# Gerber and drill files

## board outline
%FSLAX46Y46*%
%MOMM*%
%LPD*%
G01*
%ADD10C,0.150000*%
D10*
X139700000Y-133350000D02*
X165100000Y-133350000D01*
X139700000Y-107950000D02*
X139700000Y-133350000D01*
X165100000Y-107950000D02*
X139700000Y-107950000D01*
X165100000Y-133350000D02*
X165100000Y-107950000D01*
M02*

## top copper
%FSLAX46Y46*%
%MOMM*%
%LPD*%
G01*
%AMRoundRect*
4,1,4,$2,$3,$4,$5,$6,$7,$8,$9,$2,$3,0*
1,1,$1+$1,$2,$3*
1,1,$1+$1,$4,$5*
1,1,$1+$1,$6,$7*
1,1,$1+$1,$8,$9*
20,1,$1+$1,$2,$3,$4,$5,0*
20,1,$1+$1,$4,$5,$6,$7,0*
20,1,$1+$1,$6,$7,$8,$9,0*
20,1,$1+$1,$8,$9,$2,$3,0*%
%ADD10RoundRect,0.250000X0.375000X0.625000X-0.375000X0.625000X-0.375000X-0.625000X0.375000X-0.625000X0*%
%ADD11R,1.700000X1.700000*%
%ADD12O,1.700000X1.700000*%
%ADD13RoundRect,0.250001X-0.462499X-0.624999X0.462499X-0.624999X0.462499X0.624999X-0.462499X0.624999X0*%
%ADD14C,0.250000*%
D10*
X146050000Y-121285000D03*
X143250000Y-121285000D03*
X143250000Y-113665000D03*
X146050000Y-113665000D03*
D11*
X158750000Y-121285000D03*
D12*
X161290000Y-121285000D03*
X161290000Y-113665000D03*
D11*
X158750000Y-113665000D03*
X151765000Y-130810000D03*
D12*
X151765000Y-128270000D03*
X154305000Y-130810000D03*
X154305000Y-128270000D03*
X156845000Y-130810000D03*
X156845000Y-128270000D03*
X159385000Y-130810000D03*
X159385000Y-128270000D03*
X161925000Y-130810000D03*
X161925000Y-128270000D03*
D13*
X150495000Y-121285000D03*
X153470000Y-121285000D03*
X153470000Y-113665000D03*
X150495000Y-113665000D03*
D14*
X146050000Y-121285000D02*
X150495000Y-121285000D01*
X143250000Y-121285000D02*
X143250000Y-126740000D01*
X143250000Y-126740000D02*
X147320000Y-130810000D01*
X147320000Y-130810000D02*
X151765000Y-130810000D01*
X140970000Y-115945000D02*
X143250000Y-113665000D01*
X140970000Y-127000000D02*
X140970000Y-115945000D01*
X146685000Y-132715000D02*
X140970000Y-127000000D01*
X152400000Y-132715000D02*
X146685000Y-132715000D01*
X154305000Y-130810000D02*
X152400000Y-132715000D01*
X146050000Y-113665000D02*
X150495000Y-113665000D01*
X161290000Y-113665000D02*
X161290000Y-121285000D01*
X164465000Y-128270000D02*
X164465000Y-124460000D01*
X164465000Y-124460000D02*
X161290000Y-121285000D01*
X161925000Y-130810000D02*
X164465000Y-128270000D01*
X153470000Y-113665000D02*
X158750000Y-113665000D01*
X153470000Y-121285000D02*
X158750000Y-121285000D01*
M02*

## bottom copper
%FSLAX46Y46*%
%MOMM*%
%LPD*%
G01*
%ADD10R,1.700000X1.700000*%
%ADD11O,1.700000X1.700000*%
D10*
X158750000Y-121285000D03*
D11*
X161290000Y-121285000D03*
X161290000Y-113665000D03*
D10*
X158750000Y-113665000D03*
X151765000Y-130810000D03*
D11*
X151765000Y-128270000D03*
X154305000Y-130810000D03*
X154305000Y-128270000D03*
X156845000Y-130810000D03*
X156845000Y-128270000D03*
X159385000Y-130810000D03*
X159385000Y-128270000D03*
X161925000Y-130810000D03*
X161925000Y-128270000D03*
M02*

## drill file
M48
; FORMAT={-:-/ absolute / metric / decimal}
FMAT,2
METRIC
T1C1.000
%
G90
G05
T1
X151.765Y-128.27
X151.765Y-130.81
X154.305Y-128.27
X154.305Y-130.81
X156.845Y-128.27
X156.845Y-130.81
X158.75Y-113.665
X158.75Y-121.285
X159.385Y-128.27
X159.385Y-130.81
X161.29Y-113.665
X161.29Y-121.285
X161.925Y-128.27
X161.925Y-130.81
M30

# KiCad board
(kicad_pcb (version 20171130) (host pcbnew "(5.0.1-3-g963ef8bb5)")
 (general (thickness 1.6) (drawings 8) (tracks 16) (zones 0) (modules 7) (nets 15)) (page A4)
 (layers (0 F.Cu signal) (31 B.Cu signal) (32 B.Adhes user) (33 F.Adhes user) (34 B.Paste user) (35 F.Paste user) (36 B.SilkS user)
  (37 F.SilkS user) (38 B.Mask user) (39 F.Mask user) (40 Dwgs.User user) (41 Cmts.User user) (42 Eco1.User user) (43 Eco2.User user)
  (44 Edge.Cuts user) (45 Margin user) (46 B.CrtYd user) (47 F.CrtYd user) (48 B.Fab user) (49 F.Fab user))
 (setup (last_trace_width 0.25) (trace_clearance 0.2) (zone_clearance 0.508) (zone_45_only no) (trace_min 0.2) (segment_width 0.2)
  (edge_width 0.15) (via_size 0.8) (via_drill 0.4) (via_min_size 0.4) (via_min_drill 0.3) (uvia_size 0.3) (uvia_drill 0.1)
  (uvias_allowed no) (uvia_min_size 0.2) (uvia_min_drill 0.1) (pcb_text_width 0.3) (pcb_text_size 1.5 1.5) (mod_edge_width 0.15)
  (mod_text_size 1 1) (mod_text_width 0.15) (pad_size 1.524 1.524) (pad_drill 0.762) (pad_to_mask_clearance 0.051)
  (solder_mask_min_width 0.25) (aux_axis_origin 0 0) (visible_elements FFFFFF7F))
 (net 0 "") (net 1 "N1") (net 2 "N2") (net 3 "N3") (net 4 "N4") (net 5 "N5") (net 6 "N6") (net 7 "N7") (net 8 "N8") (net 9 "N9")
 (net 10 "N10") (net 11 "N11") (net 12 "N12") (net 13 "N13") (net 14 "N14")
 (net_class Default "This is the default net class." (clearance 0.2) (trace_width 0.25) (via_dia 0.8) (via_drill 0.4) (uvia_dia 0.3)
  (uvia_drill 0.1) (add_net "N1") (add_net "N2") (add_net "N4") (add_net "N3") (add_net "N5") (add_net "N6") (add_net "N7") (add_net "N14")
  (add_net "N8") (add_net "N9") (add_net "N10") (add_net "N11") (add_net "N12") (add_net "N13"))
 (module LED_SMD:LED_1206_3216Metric (layer F.Cu) (at 144.65 121.285 180)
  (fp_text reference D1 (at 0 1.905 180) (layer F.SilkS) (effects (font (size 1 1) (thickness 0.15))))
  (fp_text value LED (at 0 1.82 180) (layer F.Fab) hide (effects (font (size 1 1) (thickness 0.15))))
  (pad 1 smd roundrect (at -1.4 0 180) (size 1.25 1.75) (layers F.Cu F.Paste F.Mask) (roundrect_rratio 0.2) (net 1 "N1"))
  (pad 2 smd roundrect (at 1.4 0 180) (size 1.25 1.75) (layers F.Cu F.Paste F.Mask) (roundrect_rratio 0.2) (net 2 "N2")))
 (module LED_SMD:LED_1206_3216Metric (layer F.Cu) (at 144.65 113.665 180)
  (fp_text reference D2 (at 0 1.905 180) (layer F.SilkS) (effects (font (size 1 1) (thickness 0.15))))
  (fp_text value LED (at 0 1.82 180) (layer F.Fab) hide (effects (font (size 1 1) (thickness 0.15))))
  (pad 2 smd roundrect (at 1.4 0 180) (size 1.25 1.75) (layers F.Cu F.Paste F.Mask) (roundrect_rratio 0.2) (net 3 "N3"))
  (pad 1 smd roundrect (at -1.4 0 180) (size 1.25 1.75) (layers F.Cu F.Paste F.Mask) (roundrect_rratio 0.2) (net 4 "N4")))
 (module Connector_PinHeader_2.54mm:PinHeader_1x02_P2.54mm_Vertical (layer F.Cu) (at 158.75 121.285 90)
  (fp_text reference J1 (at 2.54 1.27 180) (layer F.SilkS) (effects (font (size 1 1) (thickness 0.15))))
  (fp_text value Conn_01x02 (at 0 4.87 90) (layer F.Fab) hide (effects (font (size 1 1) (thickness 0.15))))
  (pad 1 thru_hole rect (at 0 0 90) (size 1.7 1.7) (drill 1) (layers *.Cu *.Mask) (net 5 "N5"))
  (pad 2 thru_hole oval (at 0 2.54 90) (size 1.7 1.7) (drill 1) (layers *.Cu *.Mask) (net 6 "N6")))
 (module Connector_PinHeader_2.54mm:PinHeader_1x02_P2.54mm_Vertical (layer F.Cu) (at 158.75 113.665 90)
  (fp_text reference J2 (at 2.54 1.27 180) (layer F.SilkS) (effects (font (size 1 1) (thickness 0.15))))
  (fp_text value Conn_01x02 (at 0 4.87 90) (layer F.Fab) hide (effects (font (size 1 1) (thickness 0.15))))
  (pad 2 thru_hole oval (at 0 2.54 90) (size 1.7 1.7) (drill 1) (layers *.Cu *.Mask) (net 6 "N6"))
  (pad 1 thru_hole rect (at 0 0 90) (size 1.7 1.7) (drill 1) (layers *.Cu *.Mask) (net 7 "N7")))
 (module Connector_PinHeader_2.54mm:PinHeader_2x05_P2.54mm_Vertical (layer F.Cu) (at 151.765 130.81 90)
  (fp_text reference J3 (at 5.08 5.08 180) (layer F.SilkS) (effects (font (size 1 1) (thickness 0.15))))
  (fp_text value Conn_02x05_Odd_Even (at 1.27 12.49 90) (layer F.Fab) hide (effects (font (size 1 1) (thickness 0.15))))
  (pad 1 thru_hole rect (at 0 0 90) (size 1.7 1.7) (drill 1) (layers *.Cu *.Mask) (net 2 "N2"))
  (pad 2 thru_hole oval (at 2.54 0 90) (size 1.7 1.7) (drill 1) (layers *.Cu *.Mask) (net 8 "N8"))
  (pad 3 thru_hole oval (at 0 2.54 90) (size 1.7 1.7) (drill 1) (layers *.Cu *.Mask) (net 3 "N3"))
  (pad 4 thru_hole oval (at 2.54 2.54 90) (size 1.7 1.7) (drill 1) (layers *.Cu *.Mask) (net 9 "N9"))
  (pad 5 thru_hole oval (at 0 5.08 90) (size 1.7 1.7) (drill 1) (layers *.Cu *.Mask) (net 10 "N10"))
  (pad 6 thru_hole oval (at 2.54 5.08 90) (size 1.7 1.7) (drill 1) (layers *.Cu *.Mask) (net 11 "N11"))
  (pad 7 thru_hole oval (at 0 7.62 90) (size 1.7 1.7) (drill 1) (layers *.Cu *.Mask) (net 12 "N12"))
  (pad 8 thru_hole oval (at 2.54 7.62 90) (size 1.7 1.7) (drill 1) (layers *.Cu *.Mask) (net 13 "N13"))
  (pad 9 thru_hole oval (at 0 10.16 90) (size 1.7 1.7) (drill 1) (layers *.Cu *.Mask) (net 6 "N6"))
  (pad 10 thru_hole oval (at 2.54 10.16 90) (size 1.7 1.7) (drill 1) (layers *.Cu *.Mask) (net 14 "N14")))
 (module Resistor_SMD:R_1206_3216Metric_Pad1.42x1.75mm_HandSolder (layer F.Cu) (at 151.9825 121.285)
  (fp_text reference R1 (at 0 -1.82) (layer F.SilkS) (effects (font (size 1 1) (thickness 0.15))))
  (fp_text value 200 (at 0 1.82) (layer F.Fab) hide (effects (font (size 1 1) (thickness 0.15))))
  (pad 1 smd roundrect (at -1.4875 0) (size 1.425 1.75) (layers F.Cu F.Paste F.Mask) (roundrect_rratio 0.175439) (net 1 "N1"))
  (pad 2 smd roundrect (at 1.4875 0) (size 1.425 1.75) (layers F.Cu F.Paste F.Mask) (roundrect_rratio 0.175439) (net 5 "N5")))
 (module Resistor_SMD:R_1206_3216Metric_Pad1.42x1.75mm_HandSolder (layer F.Cu) (at 151.9825 113.665)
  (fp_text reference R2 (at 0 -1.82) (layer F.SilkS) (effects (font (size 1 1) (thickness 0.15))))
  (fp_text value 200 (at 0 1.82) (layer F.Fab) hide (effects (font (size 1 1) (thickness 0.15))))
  (pad 2 smd roundrect (at 1.4875 0) (size 1.425 1.75) (layers F.Cu F.Paste F.Mask) (roundrect_rratio 0.175439) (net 7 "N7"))
  (pad 1 smd roundrect (at -1.4875 0) (size 1.425 1.75) (layers F.Cu F.Paste F.Mask) (roundrect_rratio 0.175439) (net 4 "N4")))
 (gr_line (start 139.7 133.35) (end 165.1 133.35) (layer Edge.Cuts) (width 0.15))
 (gr_line (start 139.7 107.95) (end 139.7 133.35) (layer Edge.Cuts) (width 0.15))
 (gr_line (start 165.1 107.95) (end 139.7 107.95) (layer Edge.Cuts) (width 0.15))
 (gr_line (start 165.1 133.35) (end 165.1 107.95) (layer Edge.Cuts) (width 0.15))
 (segment (start 146.05 121.285) (end 150.495 121.285) (width 0.25) (layer F.Cu) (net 1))
 (segment (start 143.25 121.285) (end 143.25 126.74) (width 0.25) (layer F.Cu) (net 2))
 (segment (start 143.25 126.74) (end 147.32 130.81) (width 0.25) (layer F.Cu) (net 2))
 (segment (start 147.32 130.81) (end 151.765 130.81) (width 0.25) (layer F.Cu) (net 2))
 (segment (start 140.97 115.945) (end 143.25 113.665) (width 0.25) (layer F.Cu) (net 3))
 (segment (start 140.97 127) (end 140.97 115.945) (width 0.25) (layer F.Cu) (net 3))
 (segment (start 146.685 132.715) (end 140.97 127) (width 0.25) (layer F.Cu) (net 3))
 (segment (start 152.4 132.715) (end 146.685 132.715) (width 0.25) (layer F.Cu) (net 3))
 (segment (start 154.305 130.81) (end 152.4 132.715) (width 0.25) (layer F.Cu) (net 3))
 (segment (start 146.05 113.665) (end 150.495 113.665) (width 0.25) (layer F.Cu) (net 4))
 (segment (start 161.29 113.665) (end 161.29 121.285) (width 0.25) (layer F.Cu) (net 6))
 (segment (start 164.465 128.27) (end 164.465 124.46) (width 0.25) (layer F.Cu) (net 6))
 (segment (start 164.465 124.46) (end 161.29 121.285) (width 0.25) (layer F.Cu) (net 6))
 (segment (start 161.925 130.81) (end 164.465 128.27) (width 0.25) (layer F.Cu) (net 6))
 (segment (start 153.47 113.665) (end 158.75 113.665) (width 0.25) (layer F.Cu) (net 7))
 (segment (start 153.47 121.285) (end 158.75 121.285) (width 0.25) (layer F.Cu) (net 5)))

